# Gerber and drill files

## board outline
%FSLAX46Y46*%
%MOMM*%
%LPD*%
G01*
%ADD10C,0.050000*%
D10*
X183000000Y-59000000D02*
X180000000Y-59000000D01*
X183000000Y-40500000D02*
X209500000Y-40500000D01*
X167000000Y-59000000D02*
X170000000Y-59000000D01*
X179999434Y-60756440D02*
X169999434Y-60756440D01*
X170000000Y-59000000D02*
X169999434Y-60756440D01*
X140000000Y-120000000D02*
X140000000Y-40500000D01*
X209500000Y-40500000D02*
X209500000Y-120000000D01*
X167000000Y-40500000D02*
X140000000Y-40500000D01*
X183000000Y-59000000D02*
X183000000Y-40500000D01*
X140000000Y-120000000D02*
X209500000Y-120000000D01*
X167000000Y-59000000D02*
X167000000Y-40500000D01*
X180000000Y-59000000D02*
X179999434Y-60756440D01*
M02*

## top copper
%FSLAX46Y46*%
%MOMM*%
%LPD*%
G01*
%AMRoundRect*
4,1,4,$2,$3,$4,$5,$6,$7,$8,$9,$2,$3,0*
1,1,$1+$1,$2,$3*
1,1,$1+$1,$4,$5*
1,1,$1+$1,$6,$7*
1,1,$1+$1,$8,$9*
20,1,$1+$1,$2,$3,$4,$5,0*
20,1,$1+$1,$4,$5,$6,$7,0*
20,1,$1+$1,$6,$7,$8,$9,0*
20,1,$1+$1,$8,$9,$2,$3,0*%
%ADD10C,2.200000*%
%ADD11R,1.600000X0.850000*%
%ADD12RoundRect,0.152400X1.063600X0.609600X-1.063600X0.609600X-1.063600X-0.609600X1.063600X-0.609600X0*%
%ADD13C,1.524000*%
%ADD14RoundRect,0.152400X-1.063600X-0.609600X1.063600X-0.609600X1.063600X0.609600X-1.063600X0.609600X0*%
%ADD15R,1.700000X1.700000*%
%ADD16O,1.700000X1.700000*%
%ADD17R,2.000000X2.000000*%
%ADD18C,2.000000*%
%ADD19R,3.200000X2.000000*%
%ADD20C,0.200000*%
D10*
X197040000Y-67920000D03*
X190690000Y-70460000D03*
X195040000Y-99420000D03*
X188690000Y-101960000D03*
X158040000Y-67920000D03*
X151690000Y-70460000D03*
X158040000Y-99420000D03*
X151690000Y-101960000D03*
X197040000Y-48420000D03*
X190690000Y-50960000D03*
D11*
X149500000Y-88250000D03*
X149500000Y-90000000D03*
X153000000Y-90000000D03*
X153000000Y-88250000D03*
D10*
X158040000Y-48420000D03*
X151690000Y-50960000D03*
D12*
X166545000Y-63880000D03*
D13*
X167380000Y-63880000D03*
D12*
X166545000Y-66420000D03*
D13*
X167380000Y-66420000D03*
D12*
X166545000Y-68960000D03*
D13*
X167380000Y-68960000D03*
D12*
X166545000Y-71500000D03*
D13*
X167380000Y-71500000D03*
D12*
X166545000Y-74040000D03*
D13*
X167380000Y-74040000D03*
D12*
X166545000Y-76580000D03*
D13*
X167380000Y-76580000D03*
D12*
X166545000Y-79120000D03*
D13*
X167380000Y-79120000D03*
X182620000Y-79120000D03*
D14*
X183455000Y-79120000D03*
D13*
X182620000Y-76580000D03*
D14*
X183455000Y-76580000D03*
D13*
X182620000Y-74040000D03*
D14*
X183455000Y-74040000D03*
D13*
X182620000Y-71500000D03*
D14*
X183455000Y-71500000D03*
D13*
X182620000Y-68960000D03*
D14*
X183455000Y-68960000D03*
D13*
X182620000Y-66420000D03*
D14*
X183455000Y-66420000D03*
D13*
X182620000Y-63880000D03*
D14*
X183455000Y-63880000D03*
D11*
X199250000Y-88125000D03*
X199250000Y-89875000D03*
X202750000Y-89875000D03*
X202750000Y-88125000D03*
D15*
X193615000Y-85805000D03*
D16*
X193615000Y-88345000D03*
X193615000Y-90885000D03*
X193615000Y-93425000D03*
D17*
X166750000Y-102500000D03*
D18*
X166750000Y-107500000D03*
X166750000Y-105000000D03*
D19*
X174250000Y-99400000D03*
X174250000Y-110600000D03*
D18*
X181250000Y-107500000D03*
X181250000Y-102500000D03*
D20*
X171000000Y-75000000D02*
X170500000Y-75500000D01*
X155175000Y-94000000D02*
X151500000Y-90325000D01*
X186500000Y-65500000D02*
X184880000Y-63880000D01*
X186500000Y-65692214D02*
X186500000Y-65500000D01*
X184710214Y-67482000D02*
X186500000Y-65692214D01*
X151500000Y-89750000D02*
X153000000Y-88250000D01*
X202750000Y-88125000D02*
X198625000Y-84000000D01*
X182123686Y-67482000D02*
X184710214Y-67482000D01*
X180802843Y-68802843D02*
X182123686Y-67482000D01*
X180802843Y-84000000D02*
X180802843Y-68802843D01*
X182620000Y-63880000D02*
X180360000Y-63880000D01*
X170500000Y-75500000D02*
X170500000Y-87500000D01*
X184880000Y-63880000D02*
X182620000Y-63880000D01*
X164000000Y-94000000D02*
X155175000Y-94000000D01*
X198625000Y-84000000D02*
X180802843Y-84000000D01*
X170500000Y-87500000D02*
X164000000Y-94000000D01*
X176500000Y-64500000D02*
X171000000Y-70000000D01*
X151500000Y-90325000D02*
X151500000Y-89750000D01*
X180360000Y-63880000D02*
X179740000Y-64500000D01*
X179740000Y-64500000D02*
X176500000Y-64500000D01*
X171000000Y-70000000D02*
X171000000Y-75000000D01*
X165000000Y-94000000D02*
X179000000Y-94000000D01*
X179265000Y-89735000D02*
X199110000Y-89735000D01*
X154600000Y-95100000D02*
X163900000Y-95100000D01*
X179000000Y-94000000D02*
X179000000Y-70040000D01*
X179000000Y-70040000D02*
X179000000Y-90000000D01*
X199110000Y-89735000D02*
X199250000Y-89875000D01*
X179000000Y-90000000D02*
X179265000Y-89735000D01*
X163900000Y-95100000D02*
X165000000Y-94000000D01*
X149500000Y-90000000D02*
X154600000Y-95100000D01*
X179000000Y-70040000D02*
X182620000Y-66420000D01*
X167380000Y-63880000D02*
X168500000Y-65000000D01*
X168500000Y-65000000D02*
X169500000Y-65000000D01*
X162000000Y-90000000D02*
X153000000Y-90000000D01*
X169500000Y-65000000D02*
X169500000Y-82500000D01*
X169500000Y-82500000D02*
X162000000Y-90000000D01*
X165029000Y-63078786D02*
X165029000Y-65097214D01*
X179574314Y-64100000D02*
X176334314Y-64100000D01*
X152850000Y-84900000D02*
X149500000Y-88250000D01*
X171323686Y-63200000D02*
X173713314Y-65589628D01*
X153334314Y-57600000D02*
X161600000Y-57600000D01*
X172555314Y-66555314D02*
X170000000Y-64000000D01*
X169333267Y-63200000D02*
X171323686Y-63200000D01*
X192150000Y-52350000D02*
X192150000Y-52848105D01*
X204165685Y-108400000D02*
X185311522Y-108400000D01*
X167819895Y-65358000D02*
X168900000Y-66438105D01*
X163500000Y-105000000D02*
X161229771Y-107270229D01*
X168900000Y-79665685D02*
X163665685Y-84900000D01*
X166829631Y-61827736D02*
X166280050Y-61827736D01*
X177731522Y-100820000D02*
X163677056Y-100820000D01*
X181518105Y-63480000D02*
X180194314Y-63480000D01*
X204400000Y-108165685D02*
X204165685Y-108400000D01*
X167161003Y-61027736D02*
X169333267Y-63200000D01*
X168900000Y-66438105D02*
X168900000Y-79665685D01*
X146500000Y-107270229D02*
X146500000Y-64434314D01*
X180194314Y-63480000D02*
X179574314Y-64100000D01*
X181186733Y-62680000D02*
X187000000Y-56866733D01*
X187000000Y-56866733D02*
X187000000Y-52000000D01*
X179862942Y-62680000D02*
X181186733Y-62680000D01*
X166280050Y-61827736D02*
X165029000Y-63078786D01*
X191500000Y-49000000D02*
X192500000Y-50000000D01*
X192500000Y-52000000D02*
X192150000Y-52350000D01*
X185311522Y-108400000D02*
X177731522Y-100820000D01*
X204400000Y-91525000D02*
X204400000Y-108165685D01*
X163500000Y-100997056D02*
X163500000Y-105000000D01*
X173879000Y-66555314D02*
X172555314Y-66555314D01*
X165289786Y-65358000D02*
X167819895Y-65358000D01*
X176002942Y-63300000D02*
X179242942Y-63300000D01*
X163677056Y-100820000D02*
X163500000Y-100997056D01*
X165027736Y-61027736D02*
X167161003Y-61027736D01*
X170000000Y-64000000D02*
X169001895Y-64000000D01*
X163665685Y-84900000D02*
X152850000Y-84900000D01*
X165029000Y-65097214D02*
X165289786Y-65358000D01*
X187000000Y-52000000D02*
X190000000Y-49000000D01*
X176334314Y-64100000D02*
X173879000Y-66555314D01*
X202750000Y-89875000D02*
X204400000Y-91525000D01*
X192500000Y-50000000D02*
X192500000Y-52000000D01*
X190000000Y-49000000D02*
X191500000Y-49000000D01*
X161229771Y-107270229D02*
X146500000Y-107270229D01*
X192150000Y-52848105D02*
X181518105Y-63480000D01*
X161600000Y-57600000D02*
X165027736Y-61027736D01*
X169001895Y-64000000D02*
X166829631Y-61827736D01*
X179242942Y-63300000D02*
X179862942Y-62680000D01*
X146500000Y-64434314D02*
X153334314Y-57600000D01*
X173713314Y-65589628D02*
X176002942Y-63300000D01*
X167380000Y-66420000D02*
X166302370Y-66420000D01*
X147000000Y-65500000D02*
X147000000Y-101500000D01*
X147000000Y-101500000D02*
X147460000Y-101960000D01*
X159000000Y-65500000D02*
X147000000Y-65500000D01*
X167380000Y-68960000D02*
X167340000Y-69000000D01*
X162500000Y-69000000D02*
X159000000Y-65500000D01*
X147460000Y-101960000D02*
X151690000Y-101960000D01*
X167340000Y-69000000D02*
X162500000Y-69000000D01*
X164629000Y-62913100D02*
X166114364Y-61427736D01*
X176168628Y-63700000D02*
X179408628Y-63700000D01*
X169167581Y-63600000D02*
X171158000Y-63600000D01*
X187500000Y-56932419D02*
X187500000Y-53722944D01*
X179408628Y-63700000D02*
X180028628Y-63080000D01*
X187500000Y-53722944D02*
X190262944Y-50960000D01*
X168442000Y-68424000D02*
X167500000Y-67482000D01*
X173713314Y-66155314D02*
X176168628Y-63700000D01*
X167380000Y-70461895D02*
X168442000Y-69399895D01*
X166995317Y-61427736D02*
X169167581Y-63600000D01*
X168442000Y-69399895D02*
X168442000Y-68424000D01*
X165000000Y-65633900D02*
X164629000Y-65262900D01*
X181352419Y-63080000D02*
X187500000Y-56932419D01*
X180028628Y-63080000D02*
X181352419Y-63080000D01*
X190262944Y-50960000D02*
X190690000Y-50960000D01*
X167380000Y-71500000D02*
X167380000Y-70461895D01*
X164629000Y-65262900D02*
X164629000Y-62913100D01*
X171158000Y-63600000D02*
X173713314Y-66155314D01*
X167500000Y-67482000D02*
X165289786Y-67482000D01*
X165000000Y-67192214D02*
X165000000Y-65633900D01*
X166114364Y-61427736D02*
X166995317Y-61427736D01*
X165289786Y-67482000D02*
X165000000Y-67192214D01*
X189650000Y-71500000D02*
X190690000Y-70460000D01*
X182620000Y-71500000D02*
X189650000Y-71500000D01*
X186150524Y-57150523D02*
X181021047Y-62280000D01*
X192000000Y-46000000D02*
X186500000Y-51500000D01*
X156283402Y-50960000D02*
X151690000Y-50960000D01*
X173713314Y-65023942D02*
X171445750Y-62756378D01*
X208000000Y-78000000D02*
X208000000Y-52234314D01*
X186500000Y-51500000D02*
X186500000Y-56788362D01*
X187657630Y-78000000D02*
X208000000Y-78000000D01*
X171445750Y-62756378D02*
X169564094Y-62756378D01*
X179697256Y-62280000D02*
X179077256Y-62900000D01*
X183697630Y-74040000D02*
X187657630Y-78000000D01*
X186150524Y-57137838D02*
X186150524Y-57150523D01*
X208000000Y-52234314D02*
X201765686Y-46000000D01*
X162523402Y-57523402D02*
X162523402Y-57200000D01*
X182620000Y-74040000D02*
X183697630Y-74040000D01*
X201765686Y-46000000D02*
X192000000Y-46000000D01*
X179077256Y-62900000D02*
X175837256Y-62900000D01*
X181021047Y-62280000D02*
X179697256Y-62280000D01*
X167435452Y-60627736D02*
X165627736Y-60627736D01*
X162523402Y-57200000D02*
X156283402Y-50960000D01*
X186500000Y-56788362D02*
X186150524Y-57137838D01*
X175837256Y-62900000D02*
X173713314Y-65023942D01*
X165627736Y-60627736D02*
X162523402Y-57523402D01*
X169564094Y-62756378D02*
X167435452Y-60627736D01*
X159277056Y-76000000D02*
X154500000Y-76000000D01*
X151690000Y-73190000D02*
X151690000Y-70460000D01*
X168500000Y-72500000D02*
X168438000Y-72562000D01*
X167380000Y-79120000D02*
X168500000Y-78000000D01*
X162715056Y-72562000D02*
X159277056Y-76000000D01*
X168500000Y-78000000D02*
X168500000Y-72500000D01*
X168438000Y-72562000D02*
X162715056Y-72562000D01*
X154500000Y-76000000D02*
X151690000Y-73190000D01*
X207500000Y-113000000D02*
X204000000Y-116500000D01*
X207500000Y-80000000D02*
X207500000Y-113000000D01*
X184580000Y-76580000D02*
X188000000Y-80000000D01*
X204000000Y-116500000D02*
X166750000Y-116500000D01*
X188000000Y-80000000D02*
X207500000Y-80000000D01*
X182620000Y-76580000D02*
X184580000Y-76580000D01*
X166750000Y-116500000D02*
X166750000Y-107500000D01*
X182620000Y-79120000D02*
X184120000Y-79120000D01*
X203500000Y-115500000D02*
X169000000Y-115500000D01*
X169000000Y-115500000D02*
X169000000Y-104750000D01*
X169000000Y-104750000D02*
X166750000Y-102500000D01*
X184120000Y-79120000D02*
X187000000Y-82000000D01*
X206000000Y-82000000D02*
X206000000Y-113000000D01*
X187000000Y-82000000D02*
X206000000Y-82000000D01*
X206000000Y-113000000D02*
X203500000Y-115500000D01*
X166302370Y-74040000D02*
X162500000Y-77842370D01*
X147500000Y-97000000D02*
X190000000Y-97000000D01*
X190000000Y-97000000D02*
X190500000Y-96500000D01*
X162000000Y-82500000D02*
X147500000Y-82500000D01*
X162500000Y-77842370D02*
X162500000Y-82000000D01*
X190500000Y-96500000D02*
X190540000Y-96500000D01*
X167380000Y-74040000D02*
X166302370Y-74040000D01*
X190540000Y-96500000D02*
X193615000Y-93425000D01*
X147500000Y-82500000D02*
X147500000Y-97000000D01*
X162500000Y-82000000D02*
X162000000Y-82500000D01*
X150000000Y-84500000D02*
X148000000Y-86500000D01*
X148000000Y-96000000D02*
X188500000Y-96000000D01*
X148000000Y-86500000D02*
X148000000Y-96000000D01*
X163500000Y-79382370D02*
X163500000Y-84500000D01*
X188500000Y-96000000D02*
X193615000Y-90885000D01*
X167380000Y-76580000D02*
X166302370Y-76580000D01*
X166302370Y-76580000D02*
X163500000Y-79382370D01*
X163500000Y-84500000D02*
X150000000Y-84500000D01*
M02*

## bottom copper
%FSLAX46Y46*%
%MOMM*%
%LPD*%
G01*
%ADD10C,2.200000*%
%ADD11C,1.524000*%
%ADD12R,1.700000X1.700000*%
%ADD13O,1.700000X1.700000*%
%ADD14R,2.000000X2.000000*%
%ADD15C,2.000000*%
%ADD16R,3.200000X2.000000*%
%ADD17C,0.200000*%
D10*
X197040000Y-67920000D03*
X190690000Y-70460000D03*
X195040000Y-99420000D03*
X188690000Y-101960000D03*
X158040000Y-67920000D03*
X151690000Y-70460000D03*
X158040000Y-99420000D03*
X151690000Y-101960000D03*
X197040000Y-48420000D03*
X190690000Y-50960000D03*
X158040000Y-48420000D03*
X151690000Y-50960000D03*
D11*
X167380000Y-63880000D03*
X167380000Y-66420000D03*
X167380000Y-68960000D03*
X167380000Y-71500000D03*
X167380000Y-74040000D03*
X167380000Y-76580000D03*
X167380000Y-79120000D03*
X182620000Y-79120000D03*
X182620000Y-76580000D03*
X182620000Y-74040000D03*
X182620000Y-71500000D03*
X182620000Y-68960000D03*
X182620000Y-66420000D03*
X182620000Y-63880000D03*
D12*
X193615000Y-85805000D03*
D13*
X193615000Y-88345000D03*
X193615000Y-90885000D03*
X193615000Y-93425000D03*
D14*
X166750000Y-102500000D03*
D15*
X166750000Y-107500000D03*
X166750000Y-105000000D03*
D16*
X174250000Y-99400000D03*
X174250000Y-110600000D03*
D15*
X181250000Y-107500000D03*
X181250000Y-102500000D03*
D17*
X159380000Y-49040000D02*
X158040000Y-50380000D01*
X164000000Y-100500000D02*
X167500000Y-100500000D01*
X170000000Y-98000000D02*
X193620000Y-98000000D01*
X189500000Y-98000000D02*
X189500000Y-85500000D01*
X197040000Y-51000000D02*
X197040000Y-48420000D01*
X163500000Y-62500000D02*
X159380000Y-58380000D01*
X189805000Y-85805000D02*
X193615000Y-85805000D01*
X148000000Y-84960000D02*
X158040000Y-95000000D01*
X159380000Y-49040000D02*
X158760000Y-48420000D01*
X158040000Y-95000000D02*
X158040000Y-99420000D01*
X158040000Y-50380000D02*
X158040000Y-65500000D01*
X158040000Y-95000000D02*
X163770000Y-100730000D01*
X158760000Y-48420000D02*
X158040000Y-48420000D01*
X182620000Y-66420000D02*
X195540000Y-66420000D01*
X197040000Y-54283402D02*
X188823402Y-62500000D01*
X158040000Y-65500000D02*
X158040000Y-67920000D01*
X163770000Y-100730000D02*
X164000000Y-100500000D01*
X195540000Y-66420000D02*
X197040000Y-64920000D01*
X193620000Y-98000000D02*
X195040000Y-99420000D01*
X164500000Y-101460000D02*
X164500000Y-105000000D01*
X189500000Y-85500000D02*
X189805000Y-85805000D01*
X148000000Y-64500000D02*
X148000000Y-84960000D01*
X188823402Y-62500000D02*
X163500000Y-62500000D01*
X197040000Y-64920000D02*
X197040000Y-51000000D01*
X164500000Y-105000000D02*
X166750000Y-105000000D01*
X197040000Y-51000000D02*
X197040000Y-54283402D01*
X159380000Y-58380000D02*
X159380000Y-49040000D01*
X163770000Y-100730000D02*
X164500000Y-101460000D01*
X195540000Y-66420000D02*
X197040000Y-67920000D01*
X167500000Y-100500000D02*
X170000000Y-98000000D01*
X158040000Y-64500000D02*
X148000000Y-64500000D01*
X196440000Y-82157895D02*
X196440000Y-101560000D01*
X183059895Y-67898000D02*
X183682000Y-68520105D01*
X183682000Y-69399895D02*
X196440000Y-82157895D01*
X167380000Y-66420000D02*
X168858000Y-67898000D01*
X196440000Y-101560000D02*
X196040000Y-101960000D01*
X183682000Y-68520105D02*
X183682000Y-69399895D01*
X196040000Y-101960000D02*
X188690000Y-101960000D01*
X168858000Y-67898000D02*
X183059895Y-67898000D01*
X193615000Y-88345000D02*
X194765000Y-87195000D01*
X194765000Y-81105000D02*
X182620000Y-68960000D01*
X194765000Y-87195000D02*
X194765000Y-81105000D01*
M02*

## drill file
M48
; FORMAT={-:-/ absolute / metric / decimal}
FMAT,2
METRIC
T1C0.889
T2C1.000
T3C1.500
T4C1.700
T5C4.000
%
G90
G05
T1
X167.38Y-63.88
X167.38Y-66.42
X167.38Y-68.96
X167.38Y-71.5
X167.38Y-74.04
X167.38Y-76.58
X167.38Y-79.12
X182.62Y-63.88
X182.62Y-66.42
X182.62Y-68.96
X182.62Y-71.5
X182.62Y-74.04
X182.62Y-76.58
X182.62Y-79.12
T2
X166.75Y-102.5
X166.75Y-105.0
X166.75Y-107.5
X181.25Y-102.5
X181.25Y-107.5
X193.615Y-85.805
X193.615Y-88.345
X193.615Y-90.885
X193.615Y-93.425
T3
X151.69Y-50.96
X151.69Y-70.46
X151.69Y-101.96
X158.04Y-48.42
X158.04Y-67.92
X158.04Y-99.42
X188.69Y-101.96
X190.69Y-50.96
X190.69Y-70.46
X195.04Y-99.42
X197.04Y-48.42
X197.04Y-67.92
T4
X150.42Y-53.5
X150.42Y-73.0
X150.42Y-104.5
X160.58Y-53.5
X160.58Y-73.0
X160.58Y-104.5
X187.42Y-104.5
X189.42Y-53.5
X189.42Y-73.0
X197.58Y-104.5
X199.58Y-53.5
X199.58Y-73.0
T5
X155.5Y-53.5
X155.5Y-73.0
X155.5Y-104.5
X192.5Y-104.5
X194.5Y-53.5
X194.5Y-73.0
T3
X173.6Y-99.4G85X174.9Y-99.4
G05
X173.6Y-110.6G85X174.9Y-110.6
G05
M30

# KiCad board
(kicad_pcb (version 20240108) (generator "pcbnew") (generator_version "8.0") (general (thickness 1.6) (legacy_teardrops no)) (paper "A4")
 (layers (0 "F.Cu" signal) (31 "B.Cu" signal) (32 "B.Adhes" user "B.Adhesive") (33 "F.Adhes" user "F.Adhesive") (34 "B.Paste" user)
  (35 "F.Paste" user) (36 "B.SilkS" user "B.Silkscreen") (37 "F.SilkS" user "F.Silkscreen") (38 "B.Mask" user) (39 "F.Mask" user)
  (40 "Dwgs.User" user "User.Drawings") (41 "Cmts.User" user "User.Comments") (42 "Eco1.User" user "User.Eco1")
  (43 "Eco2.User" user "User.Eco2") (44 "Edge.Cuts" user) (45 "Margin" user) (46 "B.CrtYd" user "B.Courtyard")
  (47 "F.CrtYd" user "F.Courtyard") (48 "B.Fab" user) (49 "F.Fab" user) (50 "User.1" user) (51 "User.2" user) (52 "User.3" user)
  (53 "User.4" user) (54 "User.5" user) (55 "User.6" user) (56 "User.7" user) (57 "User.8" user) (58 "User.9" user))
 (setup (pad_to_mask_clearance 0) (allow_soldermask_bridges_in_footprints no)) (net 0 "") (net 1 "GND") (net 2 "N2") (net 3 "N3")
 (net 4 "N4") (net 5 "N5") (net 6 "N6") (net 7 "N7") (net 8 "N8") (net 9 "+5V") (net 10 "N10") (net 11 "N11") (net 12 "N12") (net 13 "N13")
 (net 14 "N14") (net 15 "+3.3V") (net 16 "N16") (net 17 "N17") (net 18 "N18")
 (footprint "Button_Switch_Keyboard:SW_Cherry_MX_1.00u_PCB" (layer "F.Cu") (at 197.04 67.92)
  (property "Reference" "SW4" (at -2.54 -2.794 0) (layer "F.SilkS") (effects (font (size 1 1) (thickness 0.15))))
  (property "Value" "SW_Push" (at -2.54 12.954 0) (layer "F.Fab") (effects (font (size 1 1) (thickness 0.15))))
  (pad "" np_thru_hole circle (at -7.62 5.08) (size 1.7 1.7) (drill 1.7) (layers "*.Cu" "*.Mask"))
  (pad "" np_thru_hole circle (at -2.54 5.08) (size 4 4) (drill 4) (layers "*.Cu" "*.Mask"))
  (pad "" np_thru_hole circle (at 2.54 5.08) (size 1.7 1.7) (drill 1.7) (layers "*.Cu" "*.Mask"))
  (pad "1" thru_hole circle (at 0 0) (size 2.2 2.2) (drill 1.5) (layers "*.Cu" "*.Mask") (remove_unused_layers no) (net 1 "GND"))
  (pad "2" thru_hole circle (at -6.35 2.54) (size 2.2 2.2) (drill 1.5) (layers "*.Cu" "*.Mask") (remove_unused_layers no) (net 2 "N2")))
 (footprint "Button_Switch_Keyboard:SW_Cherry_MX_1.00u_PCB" (layer "F.Cu") (at 195.04 99.42)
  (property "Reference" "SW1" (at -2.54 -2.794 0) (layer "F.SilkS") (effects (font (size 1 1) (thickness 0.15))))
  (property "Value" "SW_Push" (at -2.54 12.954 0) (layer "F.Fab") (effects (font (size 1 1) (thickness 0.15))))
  (pad "" np_thru_hole circle (at -7.62 5.08) (size 1.7 1.7) (drill 1.7) (layers "*.Cu" "*.Mask"))
  (pad "" np_thru_hole circle (at -2.54 5.08) (size 4 4) (drill 4) (layers "*.Cu" "*.Mask"))
  (pad "" np_thru_hole circle (at 2.54 5.08) (size 1.7 1.7) (drill 1.7) (layers "*.Cu" "*.Mask"))
  (pad "1" thru_hole circle (at 0 0) (size 2.2 2.2) (drill 1.5) (layers "*.Cu" "*.Mask") (remove_unused_layers no) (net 1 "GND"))
  (pad "2" thru_hole circle (at -6.35 2.54) (size 2.2 2.2) (drill 1.5) (layers "*.Cu" "*.Mask") (remove_unused_layers no) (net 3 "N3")))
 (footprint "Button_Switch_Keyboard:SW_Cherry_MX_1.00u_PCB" (layer "F.Cu") (at 158.04 67.92)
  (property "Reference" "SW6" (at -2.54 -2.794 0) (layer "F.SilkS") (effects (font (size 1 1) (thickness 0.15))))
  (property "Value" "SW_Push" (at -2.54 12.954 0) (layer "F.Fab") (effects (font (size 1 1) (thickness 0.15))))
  (pad "" np_thru_hole circle (at -7.62 5.08) (size 1.7 1.7) (drill 1.7) (layers "*.Cu" "*.Mask"))
  (pad "" np_thru_hole circle (at -2.54 5.08) (size 4 4) (drill 4) (layers "*.Cu" "*.Mask"))
  (pad "" np_thru_hole circle (at 2.54 5.08) (size 1.7 1.7) (drill 1.7) (layers "*.Cu" "*.Mask"))
  (pad "1" thru_hole circle (at 0 0) (size 2.2 2.2) (drill 1.5) (layers "*.Cu" "*.Mask") (remove_unused_layers no) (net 1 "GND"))
  (pad "2" thru_hole circle (at -6.35 2.54) (size 2.2 2.2) (drill 1.5) (layers "*.Cu" "*.Mask") (remove_unused_layers no) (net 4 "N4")))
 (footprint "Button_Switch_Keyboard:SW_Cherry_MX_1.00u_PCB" (layer "F.Cu") (at 158.04 99.42)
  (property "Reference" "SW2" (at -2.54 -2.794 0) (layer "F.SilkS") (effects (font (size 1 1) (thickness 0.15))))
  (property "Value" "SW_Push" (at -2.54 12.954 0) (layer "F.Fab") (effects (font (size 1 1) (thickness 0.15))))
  (pad "" np_thru_hole circle (at -7.62 5.08) (size 1.7 1.7) (drill 1.7) (layers "*.Cu" "*.Mask"))
  (pad "" np_thru_hole circle (at -2.54 5.08) (size 4 4) (drill 4) (layers "*.Cu" "*.Mask"))
  (pad "" np_thru_hole circle (at 2.54 5.08) (size 1.7 1.7) (drill 1.7) (layers "*.Cu" "*.Mask"))
  (pad "1" thru_hole circle (at 0 0) (size 2.2 2.2) (drill 1.5) (layers "*.Cu" "*.Mask") (remove_unused_layers no) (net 1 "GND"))
  (pad "2" thru_hole circle (at -6.35 2.54) (size 2.2 2.2) (drill 1.5) (layers "*.Cu" "*.Mask") (remove_unused_layers no) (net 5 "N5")))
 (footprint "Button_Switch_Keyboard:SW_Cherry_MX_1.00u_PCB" (layer "F.Cu") (at 197.04 48.42)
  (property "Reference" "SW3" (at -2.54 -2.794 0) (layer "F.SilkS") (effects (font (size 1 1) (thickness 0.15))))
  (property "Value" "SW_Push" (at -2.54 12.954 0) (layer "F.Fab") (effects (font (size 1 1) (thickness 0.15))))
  (pad "" np_thru_hole circle (at -7.62 5.08) (size 1.7 1.7) (drill 1.7) (layers "*.Cu" "*.Mask"))
  (pad "" np_thru_hole circle (at -2.54 5.08) (size 4 4) (drill 4) (layers "*.Cu" "*.Mask"))
  (pad "" np_thru_hole circle (at 2.54 5.08) (size 1.7 1.7) (drill 1.7) (layers "*.Cu" "*.Mask"))
  (pad "1" thru_hole circle (at 0 0) (size 2.2 2.2) (drill 1.5) (layers "*.Cu" "*.Mask") (remove_unused_layers no) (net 1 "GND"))
  (pad "2" thru_hole circle (at -6.35 2.54) (size 2.2 2.2) (drill 1.5) (layers "*.Cu" "*.Mask") (remove_unused_layers no) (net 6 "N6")))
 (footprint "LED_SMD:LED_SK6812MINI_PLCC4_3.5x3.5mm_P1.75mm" (layer "F.Cu") (at 151.25 89.125)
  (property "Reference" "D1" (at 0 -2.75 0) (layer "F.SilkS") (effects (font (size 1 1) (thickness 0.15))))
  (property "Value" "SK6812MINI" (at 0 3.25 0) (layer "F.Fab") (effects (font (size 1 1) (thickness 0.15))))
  (pad "1" smd rect (at -1.75 -0.875) (size 1.6 0.85) (layers "F.Cu" "F.Paste" "F.Mask") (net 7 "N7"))
  (pad "2" smd rect (at -1.75 0.875) (size 1.6 0.85) (layers "F.Cu" "F.Paste" "F.Mask") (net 1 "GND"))
  (pad "3" smd rect (at 1.75 0.875) (size 1.6 0.85) (layers "F.Cu" "F.Paste" "F.Mask") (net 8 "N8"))
  (pad "4" smd rect (at 1.75 -0.875) (size 1.6 0.85) (layers "F.Cu" "F.Paste" "F.Mask") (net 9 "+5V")))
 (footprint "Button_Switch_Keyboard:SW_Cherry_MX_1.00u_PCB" (layer "F.Cu") (at 158.04 48.42)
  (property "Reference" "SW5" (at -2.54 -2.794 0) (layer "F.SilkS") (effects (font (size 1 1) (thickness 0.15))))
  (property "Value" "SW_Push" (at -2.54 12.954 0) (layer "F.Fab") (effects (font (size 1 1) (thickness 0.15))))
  (pad "" np_thru_hole circle (at -7.62 5.08) (size 1.7 1.7) (drill 1.7) (layers "*.Cu" "*.Mask"))
  (pad "" np_thru_hole circle (at -2.54 5.08) (size 4 4) (drill 4) (layers "*.Cu" "*.Mask"))
  (pad "" np_thru_hole circle (at 2.54 5.08) (size 1.7 1.7) (drill 1.7) (layers "*.Cu" "*.Mask"))
  (pad "1" thru_hole circle (at 0 0) (size 2.2 2.2) (drill 1.5) (layers "*.Cu" "*.Mask") (remove_unused_layers no) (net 1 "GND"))
  (pad "2" thru_hole circle (at -6.35 2.54) (size 2.2 2.2) (drill 1.5) (layers "*.Cu" "*.Mask") (remove_unused_layers no) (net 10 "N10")))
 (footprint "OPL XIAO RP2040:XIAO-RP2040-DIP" (layer "F.Cu") (at 175 71.5)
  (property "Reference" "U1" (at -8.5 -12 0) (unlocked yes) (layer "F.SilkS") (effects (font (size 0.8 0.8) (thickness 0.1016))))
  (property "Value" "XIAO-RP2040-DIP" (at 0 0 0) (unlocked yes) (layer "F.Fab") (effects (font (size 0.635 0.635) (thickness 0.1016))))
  (pad "1" smd roundrect (at -8.455 -7.62 180) (size 2.432 1.524) (layers "F.Cu" "F.Mask") (roundrect_rratio 0.1) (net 8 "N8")
   (thermal_bridge_angle 45))
  (pad "1" thru_hole circle (at -7.62 -7.62 180) (size 1.524 1.524) (drill 0.889) (layers "*.Cu" "*.Mask") (remove_unused_layers no)
   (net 8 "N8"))
  (pad "2" smd roundrect (at -8.455 -5.08 180) (size 2.432 1.524) (layers "F.Cu" "F.Mask") (roundrect_rratio 0.1) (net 3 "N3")
   (thermal_bridge_angle 45))
  (pad "2" thru_hole circle (at -7.62 -5.08 180) (size 1.524 1.524) (drill 0.889) (layers "*.Cu" "*.Mask") (remove_unused_layers no)
   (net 3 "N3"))
  (pad "3" smd roundrect (at -8.455 -2.54 180) (size 2.432 1.524) (layers "F.Cu" "F.Mask") (roundrect_rratio 0.1) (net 5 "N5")
   (thermal_bridge_angle 45))
  (pad "3" thru_hole circle (at -7.62 -2.54 180) (size 1.524 1.524) (drill 0.889) (layers "*.Cu" "*.Mask") (remove_unused_layers no)
   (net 5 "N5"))
  (pad "4" smd roundrect (at -8.455 0 180) (size 2.432 1.524) (layers "F.Cu" "F.Mask") (roundrect_rratio 0.1) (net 6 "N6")
   (thermal_bridge_angle 45))
  (pad "4" thru_hole circle (at -7.62 0 180) (size 1.524 1.524) (drill 0.889) (layers "*.Cu" "*.Mask") (remove_unused_layers no)
   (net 6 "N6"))
  (pad "5" smd roundrect (at -8.455 2.54 180) (size 2.432 1.524) (layers "F.Cu" "F.Mask") (roundrect_rratio 0.1) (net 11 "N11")
   (thermal_bridge_angle 45))
  (pad "5" thru_hole circle (at -7.62 2.54 180) (size 1.524 1.524) (drill 0.889) (layers "*.Cu" "*.Mask") (remove_unused_layers no)
   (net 11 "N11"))
  (pad "6" smd roundrect (at -8.455 5.08 180) (size 2.432 1.524) (layers "F.Cu" "F.Mask") (roundrect_rratio 0.1) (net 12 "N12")
   (thermal_bridge_angle 45))
  (pad "6" thru_hole circle (at -7.62 5.08 180) (size 1.524 1.524) (drill 0.889) (layers "*.Cu" "*.Mask") (remove_unused_layers no)
   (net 12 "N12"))
  (pad "7" smd roundrect (at -8.455 7.62 180) (size 2.432 1.524) (layers "F.Cu" "F.Mask") (roundrect_rratio 0.1) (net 4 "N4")
   (thermal_bridge_angle 45))
  (pad "7" thru_hole circle (at -7.62 7.62 180) (size 1.524 1.524) (drill 0.889) (layers "*.Cu" "*.Mask") (remove_unused_layers no)
   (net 4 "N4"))
  (pad "8" thru_hole circle (at 7.62 7.62) (size 1.524 1.524) (drill 0.889) (layers "*.Cu" "*.Mask") (remove_unused_layers no)
   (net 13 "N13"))
  (pad "8" smd roundrect (at 8.455 7.62) (size 2.432 1.524) (layers "F.Cu" "F.Mask") (roundrect_rratio 0.1) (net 13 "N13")
   (thermal_bridge_angle 45))
  (pad "9" thru_hole circle (at 7.62 5.08) (size 1.524 1.524) (drill 0.889) (layers "*.Cu" "*.Mask") (remove_unused_layers no)
   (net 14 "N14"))
  (pad "9" smd roundrect (at 8.455 5.08) (size 2.432 1.524) (layers "F.Cu" "F.Mask") (roundrect_rratio 0.1) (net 14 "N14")
   (thermal_bridge_angle 45))
  (pad "10" thru_hole circle (at 7.62 2.54) (size 1.524 1.524) (drill 0.889) (layers "*.Cu" "*.Mask") (remove_unused_layers no)
   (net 10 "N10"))
  (pad "10" smd roundrect (at 8.455 2.54) (size 2.432 1.524) (layers "F.Cu" "F.Mask") (roundrect_rratio 0.1) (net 10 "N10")
   (thermal_bridge_angle 45))
  (pad "11" thru_hole circle (at 7.62 0) (size 1.524 1.524) (drill 0.889) (layers "*.Cu" "*.Mask") (remove_unused_layers no) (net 2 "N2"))
  (pad "11" smd roundrect (at 8.455 0) (size 2.432 1.524) (layers "F.Cu" "F.Mask") (roundrect_rratio 0.1) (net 2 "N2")
   (thermal_bridge_angle 45))
  (pad "12" thru_hole circle (at 7.62 -2.54) (size 1.524 1.524) (drill 0.889) (layers "*.Cu" "*.Mask") (remove_unused_layers no)
   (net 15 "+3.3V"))
  (pad "12" smd roundrect (at 8.455 -2.54) (size 2.432 1.524) (layers "F.Cu" "F.Mask") (roundrect_rratio 0.1) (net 15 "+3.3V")
   (thermal_bridge_angle 45))
  (pad "13" thru_hole circle (at 7.62 -5.08) (size 1.524 1.524) (drill 0.889) (layers "*.Cu" "*.Mask") (remove_unused_layers no)
   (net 1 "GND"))
  (pad "13" smd roundrect (at 8.455 -5.08) (size 2.432 1.524) (layers "F.Cu" "F.Mask") (roundrect_rratio 0.1) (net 1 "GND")
   (thermal_bridge_angle 45))
  (pad "14" thru_hole circle (at 7.62 -7.62) (size 1.524 1.524) (drill 0.889) (layers "*.Cu" "*.Mask") (remove_unused_layers no)
   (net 9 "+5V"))
  (pad "14" smd roundrect (at 8.455 -7.62) (size 2.432 1.524) (layers "F.Cu" "F.Mask") (roundrect_rratio 0.1) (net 9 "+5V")
   (thermal_bridge_angle 45)))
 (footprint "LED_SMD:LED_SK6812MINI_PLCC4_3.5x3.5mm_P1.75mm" (layer "F.Cu") (at 201 89)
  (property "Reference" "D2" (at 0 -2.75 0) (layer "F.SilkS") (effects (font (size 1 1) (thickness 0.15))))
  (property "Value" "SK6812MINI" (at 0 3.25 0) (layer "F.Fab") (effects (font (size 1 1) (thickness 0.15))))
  (pad "1" smd rect (at -1.75 -0.875) (size 1.6 0.85) (layers "F.Cu" "F.Paste" "F.Mask") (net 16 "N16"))
  (pad "2" smd rect (at -1.75 0.875) (size 1.6 0.85) (layers "F.Cu" "F.Paste" "F.Mask") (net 1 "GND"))
  (pad "3" smd rect (at 1.75 0.875) (size 1.6 0.85) (layers "F.Cu" "F.Paste" "F.Mask") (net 7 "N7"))
  (pad "4" smd rect (at 1.75 -0.875) (size 1.6 0.85) (layers "F.Cu" "F.Paste" "F.Mask") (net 9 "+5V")))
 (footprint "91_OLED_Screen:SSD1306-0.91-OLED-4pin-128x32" (layer "F.Cu") (at 157.115 83.615)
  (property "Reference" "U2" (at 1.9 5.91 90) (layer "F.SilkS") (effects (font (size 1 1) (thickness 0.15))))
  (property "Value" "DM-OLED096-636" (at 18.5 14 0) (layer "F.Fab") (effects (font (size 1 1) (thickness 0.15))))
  (pad "1" thru_hole rect (at 36.5 2.19) (size 1.7 1.7) (drill 1) (layers "*.Cu" "*.Mask") (remove_unused_layers no) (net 1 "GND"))
  (pad "2" thru_hole oval (at 36.5 4.73) (size 1.7 1.7) (drill 1) (layers "*.Cu" "*.Mask") (remove_unused_layers no) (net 15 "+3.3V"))
  (pad "3" thru_hole oval (at 36.5 7.27) (size 1.7 1.7) (drill 1) (layers "*.Cu" "*.Mask") (remove_unused_layers no) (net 12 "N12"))
  (pad "4" thru_hole oval (at 36.5 9.81) (size 1.7 1.7) (drill 1) (layers "*.Cu" "*.Mask") (remove_unused_layers no) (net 11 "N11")))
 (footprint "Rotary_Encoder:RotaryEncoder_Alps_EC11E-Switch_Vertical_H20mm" (layer "F.Cu") (at 166.75 102.5)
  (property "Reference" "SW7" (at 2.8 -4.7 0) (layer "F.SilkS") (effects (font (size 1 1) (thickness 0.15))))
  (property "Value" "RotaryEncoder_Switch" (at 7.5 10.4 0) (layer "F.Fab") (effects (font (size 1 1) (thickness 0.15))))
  (pad "A" thru_hole rect (at 0 0) (size 2 2) (drill 1) (layers "*.Cu" "*.Mask") (remove_unused_layers no) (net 13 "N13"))
  (pad "B" thru_hole circle (at 0 5) (size 2 2) (drill 1) (layers "*.Cu" "*.Mask") (remove_unused_layers no) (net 14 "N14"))
  (pad "C" thru_hole circle (at 0 2.5) (size 2 2) (drill 1) (layers "*.Cu" "*.Mask") (remove_unused_layers no) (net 1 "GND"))
  (pad "MP" thru_hole rect (at 7.5 -3.1) (size 3.2 2) (drill oval 2.8 1.5) (layers "*.Cu" "*.Mask") (remove_unused_layers no))
  (pad "MP" thru_hole rect (at 7.5 8.1) (size 3.2 2) (drill oval 2.8 1.5) (layers "*.Cu" "*.Mask") (remove_unused_layers no))
  (pad "S1" thru_hole circle (at 14.5 5) (size 2 2) (drill 1) (layers "*.Cu" "*.Mask") (remove_unused_layers no) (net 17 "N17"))
  (pad "S2" thru_hole circle (at 14.5 0) (size 2 2) (drill 1) (layers "*.Cu" "*.Mask") (remove_unused_layers no) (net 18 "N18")))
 (gr_line (start 183 59) (end 180 59) (stroke (width 0.05) (type default)) (layer "Edge.Cuts"))
 (gr_line (start 183 40.5) (end 209.5 40.5) (stroke (width 0.05) (type default)) (layer "Edge.Cuts"))
 (gr_line (start 167 59) (end 170 59) (stroke (width 0.05) (type default)) (layer "Edge.Cuts"))
 (gr_line (start 179.999434 60.75644) (end 169.999434 60.75644) (stroke (width 0.05) (type default)) (layer "Edge.Cuts"))
 (gr_line (start 170 59) (end 169.999434 60.75644) (stroke (width 0.05) (type default)) (layer "Edge.Cuts"))
 (gr_line (start 140 120) (end 140 40.5) (stroke (width 0.05) (type default)) (layer "Edge.Cuts"))
 (gr_line (start 209.5 40.5) (end 209.5 120) (stroke (width 0.05) (type default)) (layer "Edge.Cuts"))
 (gr_line (start 167 40.5) (end 140 40.5) (stroke (width 0.05) (type default)) (layer "Edge.Cuts"))
 (gr_line (start 183 59) (end 183 40.5) (stroke (width 0.05) (type default)) (layer "Edge.Cuts"))
 (gr_line (start 140 120) (end 209.5 120) (stroke (width 0.05) (type default)) (layer "Edge.Cuts"))
 (gr_line (start 167 59) (end 167 40.5) (stroke (width 0.05) (type default)) (layer "Edge.Cuts"))
 (gr_line (start 180 59) (end 179.999434 60.75644) (stroke (width 0.05) (type default)) (layer "Edge.Cuts"))
 (segment (start 171 75) (end 170.5 75.5) (width 0.2) (layer "F.Cu") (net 9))
 (segment (start 155.175 94) (end 151.5 90.325) (width 0.2) (layer "F.Cu") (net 9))
 (segment (start 186.5 65.5) (end 184.88 63.88) (width 0.2) (layer "F.Cu") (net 9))
 (segment (start 186.5 65.692214) (end 186.5 65.5) (width 0.2) (layer "F.Cu") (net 9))
 (segment (start 184.710214 67.482) (end 186.5 65.692214) (width 0.2) (layer "F.Cu") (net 9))
 (segment (start 151.5 89.75) (end 153 88.25) (width 0.2) (layer "F.Cu") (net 9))
 (segment (start 202.75 88.125) (end 198.625 84) (width 0.2) (layer "F.Cu") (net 9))
 (segment (start 182.123686 67.482) (end 184.710214 67.482) (width 0.2) (layer "F.Cu") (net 9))
 (segment (start 180.802843 68.802843) (end 182.123686 67.482) (width 0.2) (layer "F.Cu") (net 9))
 (segment (start 180.802843 84) (end 180.802843 68.802843) (width 0.2) (layer "F.Cu") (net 9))
 (segment (start 182.62 63.88) (end 180.36 63.88) (width 0.2) (layer "F.Cu") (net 9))
 (segment (start 170.5 75.5) (end 170.5 87.5) (width 0.2) (layer "F.Cu") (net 9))
 (segment (start 184.88 63.88) (end 182.62 63.88) (width 0.2) (layer "F.Cu") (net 9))
 (segment (start 164 94) (end 155.175 94) (width 0.2) (layer "F.Cu") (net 9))
 (segment (start 198.625 84) (end 180.802843 84) (width 0.2) (layer "F.Cu") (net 9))
 (segment (start 170.5 87.5) (end 164 94) (width 0.2) (layer "F.Cu") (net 9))
 (segment (start 176.5 64.5) (end 171 70) (width 0.2) (layer "F.Cu") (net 9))
 (segment (start 151.5 90.325) (end 151.5 89.75) (width 0.2) (layer "F.Cu") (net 9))
 (segment (start 180.36 63.88) (end 179.74 64.5) (width 0.2) (layer "F.Cu") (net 9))
 (segment (start 179.74 64.5) (end 176.5 64.5) (width 0.2) (layer "F.Cu") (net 9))
 (segment (start 171 70) (end 171 75) (width 0.2) (layer "F.Cu") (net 9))
 (segment (start 165 94) (end 179 94) (width 0.2) (layer "F.Cu") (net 1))
 (segment (start 179.265 89.735) (end 199.11 89.735) (width 0.2) (layer "F.Cu") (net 1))
 (segment (start 154.6 95.1) (end 163.9 95.1) (width 0.2) (layer "F.Cu") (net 1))
 (segment (start 179 94) (end 179 70.04) (width 0.2) (layer "F.Cu") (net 1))
 (segment (start 179 70.04) (end 179 90) (width 0.2) (layer "F.Cu") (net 1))
 (segment (start 199.11 89.735) (end 199.25 89.875) (width 0.2) (layer "F.Cu") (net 1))
 (segment (start 179 90) (end 179.265 89.735) (width 0.2) (layer "F.Cu") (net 1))
 (segment (start 163.9 95.1) (end 165 94) (width 0.2) (layer "F.Cu") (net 1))
 (segment (start 149.5 90) (end 154.6 95.1) (width 0.2) (layer "F.Cu") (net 1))
 (segment (start 179 70.04) (end 182.62 66.42) (width 0.2) (layer "F.Cu") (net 1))
 (segment (start 159.38 49.04) (end 158.04 50.38) (width 0.2) (layer "B.Cu") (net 1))
 (segment (start 164 100.5) (end 167.5 100.5) (width 0.2) (layer "B.Cu") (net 1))
 (segment (start 170 98) (end 193.62 98) (width 0.2) (layer "B.Cu") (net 1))
 (segment (start 189.5 98) (end 189.5 85.5) (width 0.2) (layer "B.Cu") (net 1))
 (segment (start 197.04 51) (end 197.04 48.42) (width 0.2) (layer "B.Cu") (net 1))
 (segment (start 163.5 62.5) (end 159.38 58.38) (width 0.2) (layer "B.Cu") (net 1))
 (segment (start 189.805 85.805) (end 193.615 85.805) (width 0.2) (layer "B.Cu") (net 1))
 (segment (start 148 84.96) (end 158.04 95) (width 0.2) (layer "B.Cu") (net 1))
 (segment (start 159.38 49.04) (end 158.76 48.42) (width 0.2) (layer "B.Cu") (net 1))
 (segment (start 158.04 95) (end 158.04 99.42) (width 0.2) (layer "B.Cu") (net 1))
 (segment (start 158.04 50.38) (end 158.04 65.5) (width 0.2) (layer "B.Cu") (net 1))
 (segment (start 158.04 95) (end 163.77 100.73) (width 0.2) (layer "B.Cu") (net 1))
 (segment (start 158.76 48.42) (end 158.04 48.42) (width 0.2) (layer "B.Cu") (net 1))
 (segment (start 182.62 66.42) (end 195.54 66.42) (width 0.2) (layer "B.Cu") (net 1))
 (segment (start 197.04 54.283402) (end 188.823402 62.5) (width 0.2) (layer "B.Cu") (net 1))
 (segment (start 158.04 65.5) (end 158.04 67.92) (width 0.2) (layer "B.Cu") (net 1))
 (segment (start 163.77 100.73) (end 164 100.5) (width 0.2) (layer "B.Cu") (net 1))
 (segment (start 195.54 66.42) (end 197.04 64.92) (width 0.2) (layer "B.Cu") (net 1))
 (segment (start 193.62 98) (end 195.04 99.42) (width 0.2) (layer "B.Cu") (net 1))
 (segment (start 164.5 101.46) (end 164.5 105) (width 0.2) (layer "B.Cu") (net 1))
 (segment (start 189.5 85.5) (end 189.805 85.805) (width 0.2) (layer "B.Cu") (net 1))
 (segment (start 148 64.5) (end 148 84.96) (width 0.2) (layer "B.Cu") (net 1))
 (segment (start 188.823402 62.5) (end 163.5 62.5) (width 0.2) (layer "B.Cu") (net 1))
 (segment (start 197.04 64.92) (end 197.04 51) (width 0.2) (layer "B.Cu") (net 1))
 (segment (start 164.5 105) (end 166.75 105) (width 0.2) (layer "B.Cu") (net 1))
 (segment (start 197.04 51) (end 197.04 54.283402) (width 0.2) (layer "B.Cu") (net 1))
 (segment (start 159.38 58.38) (end 159.38 49.04) (width 0.2) (layer "B.Cu") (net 1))
 (segment (start 163.77 100.73) (end 164.5 101.46) (width 0.2) (layer "B.Cu") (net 1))
 (segment (start 195.54 66.42) (end 197.04 67.92) (width 0.2) (layer "B.Cu") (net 1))
 (segment (start 167.5 100.5) (end 170 98) (width 0.2) (layer "B.Cu") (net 1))
 (segment (start 158.04 64.5) (end 148 64.5) (width 0.2) (layer "B.Cu") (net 1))
 (segment (start 167.38 63.88) (end 168.5 65) (width 0.2) (layer "F.Cu") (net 8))
 (segment (start 168.5 65) (end 169.5 65) (width 0.2) (layer "F.Cu") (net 8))
 (segment (start 162 90) (end 153 90) (width 0.2) (layer "F.Cu") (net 8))
 (segment (start 169.5 65) (end 169.5 82.5) (width 0.2) (layer "F.Cu") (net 8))
 (segment (start 169.5 82.5) (end 162 90) (width 0.2) (layer "F.Cu") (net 8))
 (segment (start 165.029 63.078786) (end 165.029 65.097214) (width 0.2) (layer "F.Cu") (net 7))
 (segment (start 179.574314 64.1) (end 176.334314 64.1) (width 0.2) (layer "F.Cu") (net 7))
 (segment (start 152.85 84.9) (end 149.5 88.25) (width 0.2) (layer "F.Cu") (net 7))
 (segment (start 171.323686 63.2) (end 173.713314 65.589628) (width 0.2) (layer "F.Cu") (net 7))
 (segment (start 153.334314 57.6) (end 161.6 57.6) (width 0.2) (layer "F.Cu") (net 7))
 (segment (start 172.555314 66.555314) (end 170 64) (width 0.2) (layer "F.Cu") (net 7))
 (segment (start 169.333267 63.2) (end 171.323686 63.2) (width 0.2) (layer "F.Cu") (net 7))
 (segment (start 192.15 52.35) (end 192.15 52.848105) (width 0.2) (layer "F.Cu") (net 7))
 (segment (start 204.165685 108.4) (end 185.311522 108.4) (width 0.2) (layer "F.Cu") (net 7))
 (segment (start 167.819895 65.358) (end 168.9 66.438105) (width 0.2) (layer "F.Cu") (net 7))
 (segment (start 163.5 105) (end 161.229771 107.270229) (width 0.2) (layer "F.Cu") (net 7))
 (segment (start 168.9 79.665685) (end 163.665685 84.9) (width 0.2) (layer "F.Cu") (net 7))
 (segment (start 166.829631 61.827736) (end 166.28005 61.827736) (width 0.2) (layer "F.Cu") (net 7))
 (segment (start 177.731522 100.82) (end 163.677056 100.82) (width 0.2) (layer "F.Cu") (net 7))
 (segment (start 181.518105 63.48) (end 180.194314 63.48) (width 0.2) (layer "F.Cu") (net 7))
 (segment (start 204.4 108.165685) (end 204.165685 108.4) (width 0.2) (layer "F.Cu") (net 7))
 (segment (start 167.161003 61.027736) (end 169.333267 63.2) (width 0.2) (layer "F.Cu") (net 7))
 (segment (start 168.9 66.438105) (end 168.9 79.665685) (width 0.2) (layer "F.Cu") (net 7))
 (segment (start 146.5 107.270229) (end 146.5 64.434314) (width 0.2) (layer "F.Cu") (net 7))
 (segment (start 180.194314 63.48) (end 179.574314 64.1) (width 0.2) (layer "F.Cu") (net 7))
 (segment (start 181.186733 62.68) (end 187 56.866733) (width 0.2) (layer "F.Cu") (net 7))
 (segment (start 187 56.866733) (end 187 52) (width 0.2) (layer "F.Cu") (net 7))
 (segment (start 179.862942 62.68) (end 181.186733 62.68) (width 0.2) (layer "F.Cu") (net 7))
 (segment (start 166.28005 61.827736) (end 165.029 63.078786) (width 0.2) (layer "F.Cu") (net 7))
 (segment (start 191.5 49) (end 192.5 50) (width 0.2) (layer "F.Cu") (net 7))
 (segment (start 192.5 52) (end 192.15 52.35) (width 0.2) (layer "F.Cu") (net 7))
 (segment (start 185.311522 108.4) (end 177.731522 100.82) (width 0.2) (layer "F.Cu") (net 7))
 (segment (start 204.4 91.525) (end 204.4 108.165685) (width 0.2) (layer "F.Cu") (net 7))
 (segment (start 163.5 100.997056) (end 163.5 105) (width 0.2) (layer "F.Cu") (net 7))
 (segment (start 173.879 66.555314) (end 172.555314 66.555314) (width 0.2) (layer "F.Cu") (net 7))
 (segment (start 165.289786 65.358) (end 167.819895 65.358) (width 0.2) (layer "F.Cu") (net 7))
 (segment (start 176.002942 63.3) (end 179.242942 63.3) (width 0.2) (layer "F.Cu") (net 7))
 (segment (start 163.677056 100.82) (end 163.5 100.997056) (width 0.2) (layer "F.Cu") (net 7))
 (segment (start 165.027736 61.027736) (end 167.161003 61.027736) (width 0.2) (layer "F.Cu") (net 7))
 (segment (start 170 64) (end 169.001895 64) (width 0.2) (layer "F.Cu") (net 7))
 (segment (start 163.665685 84.9) (end 152.85 84.9) (width 0.2) (layer "F.Cu") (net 7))
 (segment (start 165.029 65.097214) (end 165.289786 65.358) (width 0.2) (layer "F.Cu") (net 7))
 (segment (start 187 52) (end 190 49) (width 0.2) (layer "F.Cu") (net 7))
 (segment (start 176.334314 64.1) (end 173.879 66.555314) (width 0.2) (layer "F.Cu") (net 7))
 (segment (start 202.75 89.875) (end 204.4 91.525) (width 0.2) (layer "F.Cu") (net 7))
 (segment (start 192.5 50) (end 192.5 52) (width 0.2) (layer "F.Cu") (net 7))
 (segment (start 190 49) (end 191.5 49) (width 0.2) (layer "F.Cu") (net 7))
 (segment (start 161.229771 107.270229) (end 146.5 107.270229) (width 0.2) (layer "F.Cu") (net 7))
 (segment (start 192.15 52.848105) (end 181.518105 63.48) (width 0.2) (layer "F.Cu") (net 7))
 (segment (start 161.6 57.6) (end 165.027736 61.027736) (width 0.2) (layer "F.Cu") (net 7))
 (segment (start 169.001895 64) (end 166.829631 61.827736) (width 0.2) (layer "F.Cu") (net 7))
 (segment (start 179.242942 63.3) (end 179.862942 62.68) (width 0.2) (layer "F.Cu") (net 7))
 (segment (start 146.5 64.434314) (end 153.334314 57.6) (width 0.2) (layer "F.Cu") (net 7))
 (segment (start 173.713314 65.589628) (end 176.002942 63.3) (width 0.2) (layer "F.Cu") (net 7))
 (segment (start 167.38 66.42) (end 166.30237 66.42) (width 0.2) (layer "F.Cu") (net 3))
 (segment (start 196.44 82.157895) (end 196.44 101.56) (width 0.2) (layer "B.Cu") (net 3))
 (segment (start 183.059895 67.898) (end 183.682 68.520105) (width 0.2) (layer "B.Cu") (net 3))
 (segment (start 183.682 69.399895) (end 196.44 82.157895) (width 0.2) (layer "B.Cu") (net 3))
 (segment (start 167.38 66.42) (end 168.858 67.898) (width 0.2) (layer "B.Cu") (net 3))
 (segment (start 196.44 101.56) (end 196.04 101.96) (width 0.2) (layer "B.Cu") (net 3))
 (segment (start 183.682 68.520105) (end 183.682 69.399895) (width 0.2) (layer "B.Cu") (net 3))
 (segment (start 196.04 101.96) (end 188.69 101.96) (width 0.2) (layer "B.Cu") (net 3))
 (segment (start 168.858 67.898) (end 183.059895 67.898) (width 0.2) (layer "B.Cu") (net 3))
 (segment (start 147 65.5) (end 147 101.5) (width 0.2) (layer "F.Cu") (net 5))
 (segment (start 147 101.5) (end 147.46 101.96) (width 0.2) (layer "F.Cu") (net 5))
 (segment (start 159 65.5) (end 147 65.5) (width 0.2) (layer "F.Cu") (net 5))
 (segment (start 167.38 68.96) (end 167.34 69) (width 0.2) (layer "F.Cu") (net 5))
 (segment (start 162.5 69) (end 159 65.5) (width 0.2) (layer "F.Cu") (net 5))
 (segment (start 147.46 101.96) (end 151.69 101.96) (width 0.2) (layer "F.Cu") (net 5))
 (segment (start 167.34 69) (end 162.5 69) (width 0.2) (layer "F.Cu") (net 5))
 (segment (start 164.629 62.9131) (end 166.114364 61.427736) (width 0.2) (layer "F.Cu") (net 6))
 (segment (start 176.168628 63.7) (end 179.408628 63.7) (width 0.2) (layer "F.Cu") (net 6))
 (segment (start 169.167581 63.6) (end 171.158 63.6) (width 0.2) (layer "F.Cu") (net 6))
 (segment (start 187.5 56.932419) (end 187.5 53.722944) (width 0.2) (layer "F.Cu") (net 6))
 (segment (start 179.408628 63.7) (end 180.028628 63.08) (width 0.2) (layer "F.Cu") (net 6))
 (segment (start 187.5 53.722944) (end 190.262944 50.96) (width 0.2) (layer "F.Cu") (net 6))
 (segment (start 168.442 68.424) (end 167.5 67.482) (width 0.2) (layer "F.Cu") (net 6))
 (segment (start 173.713314 66.155314) (end 176.168628 63.7) (width 0.2) (layer "F.Cu") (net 6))
 (segment (start 167.38 70.461895) (end 168.442 69.399895) (width 0.2) (layer "F.Cu") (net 6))
 (segment (start 166.995317 61.427736) (end 169.167581 63.6) (width 0.2) (layer "F.Cu") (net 6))
 (segment (start 168.442 69.399895) (end 168.442 68.424) (width 0.2) (layer "F.Cu") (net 6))
 (segment (start 165 65.6339) (end 164.629 65.2629) (width 0.2) (layer "F.Cu") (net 6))
 (segment (start 181.352419 63.08) (end 187.5 56.932419) (width 0.2) (layer "F.Cu") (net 6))
 (segment (start 180.028628 63.08) (end 181.352419 63.08) (width 0.2) (layer "F.Cu") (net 6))
 (segment (start 190.262944 50.96) (end 190.69 50.96) (width 0.2) (layer "F.Cu") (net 6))
 (segment (start 167.38 71.5) (end 167.38 70.461895) (width 0.2) (layer "F.Cu") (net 6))
 (segment (start 164.629 65.2629) (end 164.629 62.9131) (width 0.2) (layer "F.Cu") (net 6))
 (segment (start 171.158 63.6) (end 173.713314 66.155314) (width 0.2) (layer "F.Cu") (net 6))
 (segment (start 167.5 67.482) (end 165.289786 67.482) (width 0.2) (layer "F.Cu") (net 6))
 (segment (start 165 67.192214) (end 165 65.6339) (width 0.2) (layer "F.Cu") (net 6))
 (segment (start 166.114364 61.427736) (end 166.995317 61.427736) (width 0.2) (layer "F.Cu") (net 6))
 (segment (start 165.289786 67.482) (end 165 67.192214) (width 0.2) (layer "F.Cu") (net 6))
 (segment (start 189.65 71.5) (end 190.69 70.46) (width 0.2) (layer "F.Cu") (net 2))
 (segment (start 182.62 71.5) (end 189.65 71.5) (width 0.2) (layer "F.Cu") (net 2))
 (segment (start 186.150524 57.150523) (end 181.021047 62.28) (width 0.2) (layer "F.Cu") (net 10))
 (segment (start 192 46) (end 186.5 51.5) (width 0.2) (layer "F.Cu") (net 10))
 (segment (start 156.283402 50.96) (end 151.69 50.96) (width 0.2) (layer "F.Cu") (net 10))
 (segment (start 173.713314 65.023942) (end 171.44575 62.756378) (width 0.2) (layer "F.Cu") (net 10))
 (segment (start 208 78) (end 208 52.234314) (width 0.2) (layer "F.Cu") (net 10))
 (segment (start 186.5 51.5) (end 186.5 56.788362) (width 0.2) (layer "F.Cu") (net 10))
 (segment (start 187.65763 78) (end 208 78) (width 0.2) (layer "F.Cu") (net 10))
 (segment (start 171.44575 62.756378) (end 169.564094 62.756378) (width 0.2) (layer "F.Cu") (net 10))
 (segment (start 179.697256 62.28) (end 179.077256 62.9) (width 0.2) (layer "F.Cu") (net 10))
 (segment (start 183.69763 74.04) (end 187.65763 78) (width 0.2) (layer "F.Cu") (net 10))
 (segment (start 186.150524 57.137838) (end 186.150524 57.150523) (width 0.2) (layer "F.Cu") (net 10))
 (segment (start 208 52.234314) (end 201.765686 46) (width 0.2) (layer "F.Cu") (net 10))
 (segment (start 162.523402 57.523402) (end 162.523402 57.2) (width 0.2) (layer "F.Cu") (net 10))
 (segment (start 182.62 74.04) (end 183.69763 74.04) (width 0.2) (layer "F.Cu") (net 10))
 (segment (start 201.765686 46) (end 192 46) (width 0.2) (layer "F.Cu") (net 10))
 (segment (start 179.077256 62.9) (end 175.837256 62.9) (width 0.2) (layer "F.Cu") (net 10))
 (segment (start 181.021047 62.28) (end 179.697256 62.28) (width 0.2) (layer "F.Cu") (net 10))
 (segment (start 167.435452 60.627736) (end 165.627736 60.627736) (width 0.2) (layer "F.Cu") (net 10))
 (segment (start 162.523402 57.2) (end 156.283402 50.96) (width 0.2) (layer "F.Cu") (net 10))
 (segment (start 186.5 56.788362) (end 186.150524 57.137838) (width 0.2) (layer "F.Cu") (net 10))
 (segment (start 175.837256 62.9) (end 173.713314 65.023942) (width 0.2) (layer "F.Cu") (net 10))
 (segment (start 165.627736 60.627736) (end 162.523402 57.523402) (width 0.2) (layer "F.Cu") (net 10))
 (segment (start 169.564094 62.756378) (end 167.435452 60.627736) (width 0.2) (layer "F.Cu") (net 10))
 (segment (start 159.277056 76) (end 154.5 76) (width 0.2) (layer "F.Cu") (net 4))
 (segment (start 151.69 73.19) (end 151.69 70.46) (width 0.2) (layer "F.Cu") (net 4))
 (segment (start 168.5 72.5) (end 168.438 72.562) (width 0.2) (layer "F.Cu") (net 4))
 (segment (start 167.38 79.12) (end 168.5 78) (width 0.2) (layer "F.Cu") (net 4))
 (segment (start 162.715056 72.562) (end 159.277056 76) (width 0.2) (layer "F.Cu") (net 4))
 (segment (start 168.5 78) (end 168.5 72.5) (width 0.2) (layer "F.Cu") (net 4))
 (segment (start 168.438 72.562) (end 162.715056 72.562) (width 0.2) (layer "F.Cu") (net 4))
 (segment (start 154.5 76) (end 151.69 73.19) (width 0.2) (layer "F.Cu") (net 4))
 (segment (start 207.5 113) (end 204 116.5) (width 0.2) (layer "F.Cu") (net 14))
 (segment (start 207.5 80) (end 207.5 113) (width 0.2) (layer "F.Cu") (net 14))
 (segment (start 184.58 76.58) (end 188 80) (width 0.2) (layer "F.Cu") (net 14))
 (segment (start 204 116.5) (end 166.75 116.5) (width 0.2) (layer "F.Cu") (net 14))
 (segment (start 188 80) (end 207.5 80) (width 0.2) (layer "F.Cu") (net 14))
 (segment (start 182.62 76.58) (end 184.58 76.58) (width 0.2) (layer "F.Cu") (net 14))
 (segment (start 166.75 116.5) (end 166.75 107.5) (width 0.2) (layer "F.Cu") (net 14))
 (segment (start 182.62 79.12) (end 184.12 79.12) (width 0.2) (layer "F.Cu") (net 13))
 (segment (start 203.5 115.5) (end 169 115.5) (width 0.2) (layer "F.Cu") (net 13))
 (segment (start 169 115.5) (end 169 104.75) (width 0.2) (layer "F.Cu") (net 13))
 (segment (start 169 104.75) (end 166.75 102.5) (width 0.2) (layer "F.Cu") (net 13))
 (segment (start 184.12 79.12) (end 187 82) (width 0.2) (layer "F.Cu") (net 13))
 (segment (start 206 82) (end 206 113) (width 0.2) (layer "F.Cu") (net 13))
 (segment (start 187 82) (end 206 82) (width 0.2) (layer "F.Cu") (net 13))
 (segment (start 206 113) (end 203.5 115.5) (width 0.2) (layer "F.Cu") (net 13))
 (segment (start 166.30237 74.04) (end 162.5 77.84237) (width 0.2) (layer "F.Cu") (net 11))
 (segment (start 147.5 97) (end 190 97) (width 0.2) (layer "F.Cu") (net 11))
 (segment (start 190 97) (end 190.5 96.5) (width 0.2) (layer "F.Cu") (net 11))
 (segment (start 162 82.5) (end 147.5 82.5) (width 0.2) (layer "F.Cu") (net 11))
 (segment (start 162.5 77.84237) (end 162.5 82) (width 0.2) (layer "F.Cu") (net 11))
 (segment (start 190.5 96.5) (end 190.54 96.5) (width 0.2) (layer "F.Cu") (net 11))
 (segment (start 167.38 74.04) (end 166.30237 74.04) (width 0.2) (layer "F.Cu") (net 11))
 (segment (start 190.54 96.5) (end 193.615 93.425) (width 0.2) (layer "F.Cu") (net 11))
 (segment (start 147.5 82.5) (end 147.5 97) (width 0.2) (layer "F.Cu") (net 11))
 (segment (start 162.5 82) (end 162 82.5) (width 0.2) (layer "F.Cu") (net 11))
 (segment (start 193.615 88.345) (end 194.765 87.195) (width 0.2) (layer "B.Cu") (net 15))
 (segment (start 194.765 81.105) (end 182.62 68.96) (width 0.2) (layer "B.Cu") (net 15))
 (segment (start 194.765 87.195) (end 194.765 81.105) (width 0.2) (layer "B.Cu") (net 15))
 (segment (start 150 84.5) (end 148 86.5) (width 0.2) (layer "F.Cu") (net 12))
 (segment (start 148 96) (end 188.5 96) (width 0.2) (layer "F.Cu") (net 12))
 (segment (start 148 86.5) (end 148 96) (width 0.2) (layer "F.Cu") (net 12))
 (segment (start 163.5 79.38237) (end 163.5 84.5) (width 0.2) (layer "F.Cu") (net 12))
 (segment (start 188.5 96) (end 193.615 90.885) (width 0.2) (layer "F.Cu") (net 12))
 (segment (start 167.38 76.58) (end 166.30237 76.58) (width 0.2) (layer "F.Cu") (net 12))
 (segment (start 166.30237 76.58) (end 163.5 79.38237) (width 0.2) (layer "F.Cu") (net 12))
 (segment (start 163.5 84.5) (end 150 84.5) (width 0.2) (layer "F.Cu") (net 12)))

